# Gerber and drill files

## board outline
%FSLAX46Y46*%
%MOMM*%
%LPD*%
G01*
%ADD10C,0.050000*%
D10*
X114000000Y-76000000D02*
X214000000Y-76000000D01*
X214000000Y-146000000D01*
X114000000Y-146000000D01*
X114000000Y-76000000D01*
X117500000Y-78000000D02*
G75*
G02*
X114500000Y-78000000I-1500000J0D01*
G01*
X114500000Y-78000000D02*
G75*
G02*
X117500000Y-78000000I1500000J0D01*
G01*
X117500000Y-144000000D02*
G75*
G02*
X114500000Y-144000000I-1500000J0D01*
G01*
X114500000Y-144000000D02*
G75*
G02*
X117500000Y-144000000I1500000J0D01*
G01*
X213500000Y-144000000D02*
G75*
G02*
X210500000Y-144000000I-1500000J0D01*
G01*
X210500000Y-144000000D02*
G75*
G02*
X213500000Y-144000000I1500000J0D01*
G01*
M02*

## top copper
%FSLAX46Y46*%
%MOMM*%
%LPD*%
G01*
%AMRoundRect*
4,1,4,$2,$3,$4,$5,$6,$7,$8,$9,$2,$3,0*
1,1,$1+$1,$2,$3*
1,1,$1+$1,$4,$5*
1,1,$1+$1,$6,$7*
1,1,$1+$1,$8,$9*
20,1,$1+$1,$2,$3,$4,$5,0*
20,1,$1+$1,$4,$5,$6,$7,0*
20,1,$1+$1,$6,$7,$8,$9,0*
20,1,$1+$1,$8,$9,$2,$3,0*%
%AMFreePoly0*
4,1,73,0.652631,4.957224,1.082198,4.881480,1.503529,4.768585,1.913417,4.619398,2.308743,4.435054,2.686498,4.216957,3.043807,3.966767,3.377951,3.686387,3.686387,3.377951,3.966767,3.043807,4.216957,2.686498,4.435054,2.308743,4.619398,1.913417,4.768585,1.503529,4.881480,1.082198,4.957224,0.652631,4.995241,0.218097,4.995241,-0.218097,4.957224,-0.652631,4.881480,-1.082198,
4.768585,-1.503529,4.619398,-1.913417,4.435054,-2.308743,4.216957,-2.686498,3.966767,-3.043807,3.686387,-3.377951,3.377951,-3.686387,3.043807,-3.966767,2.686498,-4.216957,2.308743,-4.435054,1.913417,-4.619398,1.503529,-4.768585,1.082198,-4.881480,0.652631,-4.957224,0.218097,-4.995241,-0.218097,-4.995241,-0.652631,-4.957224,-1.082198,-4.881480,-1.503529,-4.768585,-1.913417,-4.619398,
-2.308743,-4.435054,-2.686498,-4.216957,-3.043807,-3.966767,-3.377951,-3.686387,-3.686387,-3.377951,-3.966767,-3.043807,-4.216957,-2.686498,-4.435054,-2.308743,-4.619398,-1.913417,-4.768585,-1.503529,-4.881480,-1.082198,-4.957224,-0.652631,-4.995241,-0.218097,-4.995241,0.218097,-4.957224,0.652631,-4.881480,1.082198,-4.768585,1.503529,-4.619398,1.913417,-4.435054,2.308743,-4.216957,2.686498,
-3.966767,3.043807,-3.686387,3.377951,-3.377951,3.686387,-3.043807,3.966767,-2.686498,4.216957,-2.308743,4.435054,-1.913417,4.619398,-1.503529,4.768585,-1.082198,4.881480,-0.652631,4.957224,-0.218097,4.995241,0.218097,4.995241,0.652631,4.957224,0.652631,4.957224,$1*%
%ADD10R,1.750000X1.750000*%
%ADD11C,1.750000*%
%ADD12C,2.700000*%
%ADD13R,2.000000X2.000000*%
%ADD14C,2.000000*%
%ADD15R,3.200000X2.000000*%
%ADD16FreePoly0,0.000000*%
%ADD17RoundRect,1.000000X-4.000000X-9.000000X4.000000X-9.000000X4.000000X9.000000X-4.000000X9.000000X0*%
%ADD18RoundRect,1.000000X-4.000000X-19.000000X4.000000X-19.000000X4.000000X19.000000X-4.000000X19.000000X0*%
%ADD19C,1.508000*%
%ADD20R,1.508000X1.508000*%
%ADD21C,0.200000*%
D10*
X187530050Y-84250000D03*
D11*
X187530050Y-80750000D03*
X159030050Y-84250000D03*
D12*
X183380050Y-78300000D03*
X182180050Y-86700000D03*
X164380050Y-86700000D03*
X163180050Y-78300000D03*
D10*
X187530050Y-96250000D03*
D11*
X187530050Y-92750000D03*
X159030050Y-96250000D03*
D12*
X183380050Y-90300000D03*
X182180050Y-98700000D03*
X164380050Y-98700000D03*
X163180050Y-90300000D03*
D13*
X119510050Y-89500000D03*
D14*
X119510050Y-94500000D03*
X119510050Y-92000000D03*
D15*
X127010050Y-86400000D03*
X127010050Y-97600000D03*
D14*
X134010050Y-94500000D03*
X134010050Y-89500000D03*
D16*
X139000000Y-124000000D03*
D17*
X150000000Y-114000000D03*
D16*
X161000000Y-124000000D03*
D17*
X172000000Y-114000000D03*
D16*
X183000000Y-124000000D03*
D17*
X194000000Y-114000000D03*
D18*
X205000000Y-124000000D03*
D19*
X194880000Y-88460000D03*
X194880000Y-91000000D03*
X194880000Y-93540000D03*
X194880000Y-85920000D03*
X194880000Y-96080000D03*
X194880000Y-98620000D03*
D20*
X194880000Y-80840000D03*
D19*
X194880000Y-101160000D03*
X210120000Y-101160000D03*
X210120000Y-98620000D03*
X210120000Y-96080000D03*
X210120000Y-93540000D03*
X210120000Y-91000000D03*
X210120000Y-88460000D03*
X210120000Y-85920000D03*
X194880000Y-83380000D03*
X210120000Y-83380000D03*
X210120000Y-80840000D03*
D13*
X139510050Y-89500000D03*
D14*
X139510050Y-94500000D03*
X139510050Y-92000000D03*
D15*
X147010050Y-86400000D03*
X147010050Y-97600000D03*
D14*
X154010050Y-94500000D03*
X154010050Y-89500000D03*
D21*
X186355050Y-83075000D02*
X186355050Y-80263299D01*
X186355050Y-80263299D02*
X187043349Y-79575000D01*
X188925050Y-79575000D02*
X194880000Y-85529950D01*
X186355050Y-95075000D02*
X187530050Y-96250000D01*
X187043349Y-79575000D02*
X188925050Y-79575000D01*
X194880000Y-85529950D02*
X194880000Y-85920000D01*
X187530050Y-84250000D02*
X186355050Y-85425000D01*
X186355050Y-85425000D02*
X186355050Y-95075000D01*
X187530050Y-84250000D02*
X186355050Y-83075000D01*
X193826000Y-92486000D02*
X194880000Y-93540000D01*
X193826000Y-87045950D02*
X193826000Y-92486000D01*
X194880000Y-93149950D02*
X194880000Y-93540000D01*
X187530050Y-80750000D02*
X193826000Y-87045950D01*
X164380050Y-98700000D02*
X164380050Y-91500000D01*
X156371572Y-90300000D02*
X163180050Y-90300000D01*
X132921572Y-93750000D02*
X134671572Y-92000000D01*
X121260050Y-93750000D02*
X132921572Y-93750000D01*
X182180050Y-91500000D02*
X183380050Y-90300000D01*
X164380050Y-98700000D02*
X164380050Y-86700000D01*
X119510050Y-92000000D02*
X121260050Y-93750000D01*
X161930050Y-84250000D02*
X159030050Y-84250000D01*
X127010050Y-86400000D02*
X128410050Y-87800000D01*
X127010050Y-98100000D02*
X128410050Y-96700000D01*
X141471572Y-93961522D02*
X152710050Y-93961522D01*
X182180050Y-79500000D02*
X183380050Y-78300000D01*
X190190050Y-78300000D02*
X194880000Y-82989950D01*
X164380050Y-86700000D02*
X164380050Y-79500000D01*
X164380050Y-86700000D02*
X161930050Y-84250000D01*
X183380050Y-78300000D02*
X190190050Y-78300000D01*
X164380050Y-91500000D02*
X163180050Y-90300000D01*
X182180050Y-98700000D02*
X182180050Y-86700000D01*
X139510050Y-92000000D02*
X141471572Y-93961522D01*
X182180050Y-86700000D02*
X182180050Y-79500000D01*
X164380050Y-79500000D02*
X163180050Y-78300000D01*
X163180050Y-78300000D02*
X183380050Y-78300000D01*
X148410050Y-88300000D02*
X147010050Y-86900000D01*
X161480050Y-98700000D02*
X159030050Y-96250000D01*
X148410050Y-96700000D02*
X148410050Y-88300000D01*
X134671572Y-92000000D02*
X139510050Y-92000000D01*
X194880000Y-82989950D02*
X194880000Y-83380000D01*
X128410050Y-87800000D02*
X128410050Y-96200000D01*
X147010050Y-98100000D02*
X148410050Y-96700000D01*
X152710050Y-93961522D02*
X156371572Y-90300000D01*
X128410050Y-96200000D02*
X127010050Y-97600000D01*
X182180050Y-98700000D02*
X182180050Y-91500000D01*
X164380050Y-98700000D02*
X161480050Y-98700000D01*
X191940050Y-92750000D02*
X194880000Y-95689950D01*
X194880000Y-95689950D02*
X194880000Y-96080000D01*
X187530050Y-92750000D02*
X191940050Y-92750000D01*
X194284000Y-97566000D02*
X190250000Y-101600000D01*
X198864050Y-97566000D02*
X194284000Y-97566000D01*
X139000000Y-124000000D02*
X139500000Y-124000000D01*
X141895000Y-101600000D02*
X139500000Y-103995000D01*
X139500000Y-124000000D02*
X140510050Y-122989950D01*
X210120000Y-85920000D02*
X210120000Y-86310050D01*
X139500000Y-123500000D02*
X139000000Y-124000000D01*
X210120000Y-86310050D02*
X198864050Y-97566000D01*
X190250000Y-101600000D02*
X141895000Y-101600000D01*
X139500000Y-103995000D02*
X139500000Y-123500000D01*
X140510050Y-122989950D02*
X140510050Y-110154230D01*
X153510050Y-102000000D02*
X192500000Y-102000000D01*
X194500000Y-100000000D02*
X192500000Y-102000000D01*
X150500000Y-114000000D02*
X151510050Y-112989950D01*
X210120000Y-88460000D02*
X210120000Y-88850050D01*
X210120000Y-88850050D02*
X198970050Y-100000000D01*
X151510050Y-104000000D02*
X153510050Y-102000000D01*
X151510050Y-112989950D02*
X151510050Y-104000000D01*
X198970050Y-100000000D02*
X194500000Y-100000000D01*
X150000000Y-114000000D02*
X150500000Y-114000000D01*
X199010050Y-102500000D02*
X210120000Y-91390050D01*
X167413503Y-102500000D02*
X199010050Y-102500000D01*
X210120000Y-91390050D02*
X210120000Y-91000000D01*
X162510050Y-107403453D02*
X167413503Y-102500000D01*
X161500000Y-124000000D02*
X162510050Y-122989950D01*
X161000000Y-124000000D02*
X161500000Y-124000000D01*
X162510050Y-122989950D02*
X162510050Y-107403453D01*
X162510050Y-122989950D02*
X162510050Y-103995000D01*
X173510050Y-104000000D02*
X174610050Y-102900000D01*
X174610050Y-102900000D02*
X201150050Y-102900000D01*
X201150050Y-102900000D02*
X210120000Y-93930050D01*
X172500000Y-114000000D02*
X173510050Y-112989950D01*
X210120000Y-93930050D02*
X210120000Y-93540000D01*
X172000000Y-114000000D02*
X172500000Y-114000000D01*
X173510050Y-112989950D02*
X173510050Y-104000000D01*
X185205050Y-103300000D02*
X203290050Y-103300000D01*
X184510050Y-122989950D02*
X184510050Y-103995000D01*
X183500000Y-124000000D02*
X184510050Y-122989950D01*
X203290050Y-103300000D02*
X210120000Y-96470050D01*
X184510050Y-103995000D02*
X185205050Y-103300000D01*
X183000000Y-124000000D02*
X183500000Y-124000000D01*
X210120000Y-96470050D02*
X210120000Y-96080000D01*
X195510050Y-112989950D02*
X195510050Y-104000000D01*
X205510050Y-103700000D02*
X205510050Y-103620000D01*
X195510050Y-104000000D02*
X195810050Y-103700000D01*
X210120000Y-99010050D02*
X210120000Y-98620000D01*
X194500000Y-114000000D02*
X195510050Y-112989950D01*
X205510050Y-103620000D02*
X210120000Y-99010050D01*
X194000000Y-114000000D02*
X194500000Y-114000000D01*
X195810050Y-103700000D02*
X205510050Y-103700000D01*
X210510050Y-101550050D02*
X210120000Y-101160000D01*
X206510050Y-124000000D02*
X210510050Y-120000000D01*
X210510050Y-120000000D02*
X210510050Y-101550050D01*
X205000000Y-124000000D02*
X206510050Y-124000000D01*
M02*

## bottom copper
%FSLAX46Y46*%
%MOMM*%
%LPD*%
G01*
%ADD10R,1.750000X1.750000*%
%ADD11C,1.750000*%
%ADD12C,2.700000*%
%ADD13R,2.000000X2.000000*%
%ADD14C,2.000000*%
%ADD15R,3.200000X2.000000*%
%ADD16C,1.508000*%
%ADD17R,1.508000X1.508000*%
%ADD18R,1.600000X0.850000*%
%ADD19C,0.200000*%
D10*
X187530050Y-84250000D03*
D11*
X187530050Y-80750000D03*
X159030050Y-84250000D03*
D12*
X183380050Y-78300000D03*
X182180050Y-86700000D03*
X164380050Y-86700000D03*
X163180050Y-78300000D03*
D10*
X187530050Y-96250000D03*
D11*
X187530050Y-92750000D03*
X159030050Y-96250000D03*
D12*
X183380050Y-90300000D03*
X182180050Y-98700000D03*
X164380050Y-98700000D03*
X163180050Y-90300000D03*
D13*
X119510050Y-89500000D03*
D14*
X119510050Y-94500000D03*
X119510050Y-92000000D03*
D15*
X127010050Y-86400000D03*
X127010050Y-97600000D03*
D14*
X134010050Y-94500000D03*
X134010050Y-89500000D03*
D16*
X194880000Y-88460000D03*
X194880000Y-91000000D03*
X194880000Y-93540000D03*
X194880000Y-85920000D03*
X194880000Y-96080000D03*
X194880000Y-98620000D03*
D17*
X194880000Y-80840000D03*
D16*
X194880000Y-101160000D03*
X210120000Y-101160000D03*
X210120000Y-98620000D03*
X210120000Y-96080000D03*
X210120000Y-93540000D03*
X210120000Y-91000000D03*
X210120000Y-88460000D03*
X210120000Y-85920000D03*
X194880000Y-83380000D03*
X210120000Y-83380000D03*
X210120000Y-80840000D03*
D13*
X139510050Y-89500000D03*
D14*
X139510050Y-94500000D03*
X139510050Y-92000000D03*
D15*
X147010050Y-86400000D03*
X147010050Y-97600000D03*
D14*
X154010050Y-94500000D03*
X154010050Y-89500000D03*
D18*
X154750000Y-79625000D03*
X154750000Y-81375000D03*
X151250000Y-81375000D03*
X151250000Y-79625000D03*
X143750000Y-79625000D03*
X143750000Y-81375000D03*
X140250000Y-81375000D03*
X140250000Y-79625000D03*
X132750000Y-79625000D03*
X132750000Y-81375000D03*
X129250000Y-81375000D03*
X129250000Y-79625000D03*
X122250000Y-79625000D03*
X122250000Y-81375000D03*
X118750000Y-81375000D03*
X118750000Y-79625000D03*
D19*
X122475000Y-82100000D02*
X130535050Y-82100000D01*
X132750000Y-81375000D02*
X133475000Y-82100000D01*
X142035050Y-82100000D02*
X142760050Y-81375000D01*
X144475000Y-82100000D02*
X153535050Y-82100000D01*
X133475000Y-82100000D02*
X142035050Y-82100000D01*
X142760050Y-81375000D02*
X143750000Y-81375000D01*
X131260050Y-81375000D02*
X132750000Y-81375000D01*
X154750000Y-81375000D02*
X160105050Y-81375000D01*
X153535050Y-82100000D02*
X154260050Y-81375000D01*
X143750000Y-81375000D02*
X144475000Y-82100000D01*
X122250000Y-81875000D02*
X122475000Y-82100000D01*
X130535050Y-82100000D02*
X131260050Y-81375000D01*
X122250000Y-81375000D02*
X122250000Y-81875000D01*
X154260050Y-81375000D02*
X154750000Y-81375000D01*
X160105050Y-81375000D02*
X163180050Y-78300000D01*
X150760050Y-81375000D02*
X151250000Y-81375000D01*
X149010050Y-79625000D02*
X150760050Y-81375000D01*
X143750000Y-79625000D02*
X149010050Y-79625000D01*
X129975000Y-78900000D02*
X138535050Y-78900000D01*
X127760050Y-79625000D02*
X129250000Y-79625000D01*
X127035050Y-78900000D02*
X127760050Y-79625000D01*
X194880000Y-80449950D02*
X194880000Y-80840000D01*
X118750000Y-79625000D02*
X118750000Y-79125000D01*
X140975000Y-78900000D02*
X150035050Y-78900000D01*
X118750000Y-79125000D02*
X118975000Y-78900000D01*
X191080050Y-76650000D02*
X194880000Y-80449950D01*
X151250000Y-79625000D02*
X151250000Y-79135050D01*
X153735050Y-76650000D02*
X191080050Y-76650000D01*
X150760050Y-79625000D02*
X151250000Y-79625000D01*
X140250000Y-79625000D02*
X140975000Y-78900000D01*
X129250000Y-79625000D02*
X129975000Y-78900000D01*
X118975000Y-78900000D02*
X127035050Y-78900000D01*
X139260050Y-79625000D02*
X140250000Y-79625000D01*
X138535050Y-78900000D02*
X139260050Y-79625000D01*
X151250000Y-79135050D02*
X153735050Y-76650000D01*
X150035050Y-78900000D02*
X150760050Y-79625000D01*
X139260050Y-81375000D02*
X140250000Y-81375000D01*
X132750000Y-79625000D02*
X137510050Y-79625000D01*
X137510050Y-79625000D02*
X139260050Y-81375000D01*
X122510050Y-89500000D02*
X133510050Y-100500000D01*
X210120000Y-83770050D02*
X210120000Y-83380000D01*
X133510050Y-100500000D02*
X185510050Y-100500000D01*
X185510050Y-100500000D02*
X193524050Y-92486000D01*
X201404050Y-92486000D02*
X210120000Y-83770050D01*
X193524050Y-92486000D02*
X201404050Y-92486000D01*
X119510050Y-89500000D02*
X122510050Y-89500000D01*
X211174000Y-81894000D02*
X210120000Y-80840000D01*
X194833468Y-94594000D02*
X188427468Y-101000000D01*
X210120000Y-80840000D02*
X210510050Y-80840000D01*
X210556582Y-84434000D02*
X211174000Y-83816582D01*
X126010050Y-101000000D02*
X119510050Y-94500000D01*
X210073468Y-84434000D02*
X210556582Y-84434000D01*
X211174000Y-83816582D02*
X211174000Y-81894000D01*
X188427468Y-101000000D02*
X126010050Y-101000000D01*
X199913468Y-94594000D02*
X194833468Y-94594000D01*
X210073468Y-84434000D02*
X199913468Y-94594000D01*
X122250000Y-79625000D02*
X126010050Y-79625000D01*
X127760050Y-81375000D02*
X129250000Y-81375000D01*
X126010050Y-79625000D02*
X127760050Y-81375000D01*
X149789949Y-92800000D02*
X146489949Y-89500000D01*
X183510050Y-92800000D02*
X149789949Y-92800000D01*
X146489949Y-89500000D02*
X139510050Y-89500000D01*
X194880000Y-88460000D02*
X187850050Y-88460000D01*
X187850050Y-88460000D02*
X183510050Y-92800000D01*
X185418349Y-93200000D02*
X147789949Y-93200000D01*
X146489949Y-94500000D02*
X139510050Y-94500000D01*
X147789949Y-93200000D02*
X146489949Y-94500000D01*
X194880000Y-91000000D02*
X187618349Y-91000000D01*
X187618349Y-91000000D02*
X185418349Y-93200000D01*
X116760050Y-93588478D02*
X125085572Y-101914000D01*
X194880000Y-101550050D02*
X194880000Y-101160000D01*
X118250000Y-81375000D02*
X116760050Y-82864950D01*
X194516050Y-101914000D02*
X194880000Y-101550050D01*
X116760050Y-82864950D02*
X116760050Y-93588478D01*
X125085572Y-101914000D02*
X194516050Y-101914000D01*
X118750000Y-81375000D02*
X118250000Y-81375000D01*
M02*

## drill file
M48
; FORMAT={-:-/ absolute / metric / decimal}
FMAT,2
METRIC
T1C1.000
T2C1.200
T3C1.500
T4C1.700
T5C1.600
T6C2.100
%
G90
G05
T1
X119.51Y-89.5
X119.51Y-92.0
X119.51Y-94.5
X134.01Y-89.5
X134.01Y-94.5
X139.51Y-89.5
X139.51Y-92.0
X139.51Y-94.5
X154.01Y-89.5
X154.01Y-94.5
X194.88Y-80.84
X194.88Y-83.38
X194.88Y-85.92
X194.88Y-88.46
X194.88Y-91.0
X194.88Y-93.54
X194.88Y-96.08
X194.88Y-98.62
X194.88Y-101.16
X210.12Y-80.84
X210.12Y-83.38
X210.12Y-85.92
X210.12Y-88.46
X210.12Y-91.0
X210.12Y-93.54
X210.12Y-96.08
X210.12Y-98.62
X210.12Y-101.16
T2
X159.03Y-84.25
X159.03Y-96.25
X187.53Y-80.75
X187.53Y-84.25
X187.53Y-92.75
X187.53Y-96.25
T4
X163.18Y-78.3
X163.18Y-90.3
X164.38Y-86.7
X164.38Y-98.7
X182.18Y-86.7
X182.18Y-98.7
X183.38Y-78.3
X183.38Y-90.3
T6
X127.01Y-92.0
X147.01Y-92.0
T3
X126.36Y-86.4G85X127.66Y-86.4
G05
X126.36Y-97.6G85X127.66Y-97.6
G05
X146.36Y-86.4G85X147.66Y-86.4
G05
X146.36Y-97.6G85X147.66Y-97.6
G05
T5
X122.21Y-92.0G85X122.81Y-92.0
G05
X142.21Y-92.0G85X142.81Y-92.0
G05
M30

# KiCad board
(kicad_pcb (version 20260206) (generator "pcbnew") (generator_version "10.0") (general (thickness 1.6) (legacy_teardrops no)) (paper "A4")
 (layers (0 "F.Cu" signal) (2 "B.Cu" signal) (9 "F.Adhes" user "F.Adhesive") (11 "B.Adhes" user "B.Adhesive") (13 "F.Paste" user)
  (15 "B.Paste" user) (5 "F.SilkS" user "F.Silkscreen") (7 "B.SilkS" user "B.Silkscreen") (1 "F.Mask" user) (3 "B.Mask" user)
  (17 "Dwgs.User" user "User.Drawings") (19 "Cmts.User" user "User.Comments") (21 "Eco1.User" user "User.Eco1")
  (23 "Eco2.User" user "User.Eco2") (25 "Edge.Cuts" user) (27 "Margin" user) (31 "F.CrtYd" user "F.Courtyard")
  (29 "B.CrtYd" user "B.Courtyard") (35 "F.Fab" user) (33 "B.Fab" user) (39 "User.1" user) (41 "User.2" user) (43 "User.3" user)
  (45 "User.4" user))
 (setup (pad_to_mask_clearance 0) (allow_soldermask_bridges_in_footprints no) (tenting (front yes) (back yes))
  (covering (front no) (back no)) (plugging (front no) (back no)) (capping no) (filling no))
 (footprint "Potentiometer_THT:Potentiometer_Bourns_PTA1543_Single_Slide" (layer "F.Cu") (at 187.53005 84.25 180)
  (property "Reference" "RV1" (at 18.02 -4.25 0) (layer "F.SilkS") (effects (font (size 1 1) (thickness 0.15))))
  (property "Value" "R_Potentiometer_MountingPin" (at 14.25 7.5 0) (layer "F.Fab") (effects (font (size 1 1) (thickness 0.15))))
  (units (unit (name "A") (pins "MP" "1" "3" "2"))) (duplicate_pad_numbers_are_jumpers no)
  (pad "1" thru_hole rect (at 0 0 180) (size 1.75 1.75) (drill 1.2) (layers "*.Cu" "*.Mask") (remove_unused_layers no) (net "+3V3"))
  (pad "2" thru_hole circle (at 0 3.5 180) (size 1.75 1.75) (drill 1.2) (layers "*.Cu" "*.Mask") (remove_unused_layers no) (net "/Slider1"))
  (pad "3" thru_hole circle (at 28.5 0 180) (size 1.75 1.75) (drill 1.2) (layers "*.Cu" "*.Mask") (remove_unused_layers no) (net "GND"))
  (pad "MP" thru_hole circle (at 4.15 5.95 180) (size 2.7 2.7) (drill 1.7) (layers "*.Cu" "*.Mask") (remove_unused_layers no) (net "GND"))
  (pad "MP" thru_hole circle (at 5.35 -2.45 180) (size 2.7 2.7) (drill 1.7) (layers "*.Cu" "*.Mask") (remove_unused_layers no) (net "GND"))
  (pad "MP" thru_hole circle (at 23.15 -2.45 180) (size 2.7 2.7) (drill 1.7) (layers "*.Cu" "*.Mask") (remove_unused_layers no) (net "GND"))
  (pad "MP" thru_hole circle (at 24.35 5.95 180) (size 2.7 2.7) (drill 1.7) (layers "*.Cu" "*.Mask") (remove_unused_layers no) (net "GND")))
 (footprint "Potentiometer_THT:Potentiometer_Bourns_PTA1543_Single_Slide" (layer "F.Cu") (at 187.53005 96.25 180)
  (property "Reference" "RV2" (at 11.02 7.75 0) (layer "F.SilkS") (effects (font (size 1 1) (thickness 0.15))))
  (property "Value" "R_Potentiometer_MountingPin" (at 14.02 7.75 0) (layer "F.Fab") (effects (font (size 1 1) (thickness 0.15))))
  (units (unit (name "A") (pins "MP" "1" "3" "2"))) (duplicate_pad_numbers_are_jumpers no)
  (pad "1" thru_hole rect (at 0 0 180) (size 1.75 1.75) (drill 1.2) (layers "*.Cu" "*.Mask") (remove_unused_layers no) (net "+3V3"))
  (pad "2" thru_hole circle (at 0 3.5 180) (size 1.75 1.75) (drill 1.2) (layers "*.Cu" "*.Mask") (remove_unused_layers no) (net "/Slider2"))
  (pad "3" thru_hole circle (at 28.5 0 180) (size 1.75 1.75) (drill 1.2) (layers "*.Cu" "*.Mask") (remove_unused_layers no) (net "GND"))
  (pad "MP" thru_hole circle (at 4.15 5.95 180) (size 2.7 2.7) (drill 1.7) (layers "*.Cu" "*.Mask") (remove_unused_layers no) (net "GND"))
  (pad "MP" thru_hole circle (at 5.35 -2.45 180) (size 2.7 2.7) (drill 1.7) (layers "*.Cu" "*.Mask") (remove_unused_layers no) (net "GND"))
  (pad "MP" thru_hole circle (at 23.15 -2.45 180) (size 2.7 2.7) (drill 1.7) (layers "*.Cu" "*.Mask") (remove_unused_layers no) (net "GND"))
  (pad "MP" thru_hole circle (at 24.35 5.95 180) (size 2.7 2.7) (drill 1.7) (layers "*.Cu" "*.Mask") (remove_unused_layers no) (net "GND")))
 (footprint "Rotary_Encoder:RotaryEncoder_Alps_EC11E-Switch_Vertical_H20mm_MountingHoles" (layer "F.Cu") (at 119.51005 89.5)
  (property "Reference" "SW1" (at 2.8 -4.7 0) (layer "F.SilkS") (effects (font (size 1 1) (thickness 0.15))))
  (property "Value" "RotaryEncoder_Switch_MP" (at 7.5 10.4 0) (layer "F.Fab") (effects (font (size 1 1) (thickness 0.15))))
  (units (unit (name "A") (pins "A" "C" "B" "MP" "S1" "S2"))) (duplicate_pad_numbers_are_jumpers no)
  (pad "" np_thru_hole oval (at 3 2.5) (size 2.2 1.6) (drill oval 2.2 1.6) (layers "*.Mask"))
  (pad "" np_thru_hole circle (at 7.5 2.5) (size 2.1 2.1) (drill 2.1) (layers "*.Mask"))
  (pad "A" thru_hole rect (at 0 0) (size 2 2) (drill 1) (layers "*.Cu" "*.Mask") (remove_unused_layers no) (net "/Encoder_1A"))
  (pad "B" thru_hole circle (at 0 5) (size 2 2) (drill 1) (layers "*.Cu" "*.Mask") (remove_unused_layers no) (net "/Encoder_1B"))
  (pad "C" thru_hole circle (at 0 2.5) (size 2 2) (drill 1) (layers "*.Cu" "*.Mask") (remove_unused_layers no) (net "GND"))
  (pad "MP" thru_hole rect (at 7.5 -3.1) (size 3.2 2) (drill oval 2.8 1.5) (layers "*.Cu" "*.Mask") (remove_unused_layers no) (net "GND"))
  (pad "MP" thru_hole rect (at 7.5 8.1) (size 3.2 2) (drill oval 2.8 1.5) (layers "*.Cu" "*.Mask") (remove_unused_layers no) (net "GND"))
  (pad "S1" thru_hole circle (at 14.5 5) (size 2 2) (drill 1) (layers "*.Cu" "*.Mask") (remove_unused_layers no)
   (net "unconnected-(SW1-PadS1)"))
  (pad "S2" thru_hole circle (at 14.5 0) (size 2 2) (drill 1) (layers "*.Cu" "*.Mask") (remove_unused_layers no)
   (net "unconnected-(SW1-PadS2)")))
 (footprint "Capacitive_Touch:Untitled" (layer "F.Cu") (at 172 100)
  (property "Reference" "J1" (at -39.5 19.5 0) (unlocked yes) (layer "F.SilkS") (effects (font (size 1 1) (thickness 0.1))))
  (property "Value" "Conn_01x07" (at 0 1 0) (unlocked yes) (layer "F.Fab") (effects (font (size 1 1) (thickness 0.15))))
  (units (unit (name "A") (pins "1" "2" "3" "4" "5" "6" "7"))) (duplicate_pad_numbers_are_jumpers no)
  (pad "1" smd custom (at -33 24) (size 10 10) (layers "F.Cu" "F.Mask") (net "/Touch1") (thermal_bridge_angle 90)
   (options (clearance outline) (anchor circle)) (primitives))
  (pad "2" smd roundrect (at -22 14) (size 10 20) (layers "F.Cu" "F.Mask") (roundrect_rratio 0.1) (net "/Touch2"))
  (pad "3" smd custom (at -11 24) (size 10 10) (layers "F.Cu" "F.Mask") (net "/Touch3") (thermal_bridge_angle 90)
   (options (clearance outline) (anchor circle)) (primitives))
  (pad "4" smd roundrect (at 0 14) (size 10 20) (layers "F.Cu" "F.Mask") (roundrect_rratio 0.1) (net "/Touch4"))
  (pad "5" smd custom (at 11 24) (size 10 10) (layers "F.Cu" "F.Mask") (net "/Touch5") (thermal_bridge_angle 90)
   (options (clearance outline) (anchor circle)) (primitives))
  (pad "6" smd roundrect (at 22 14) (size 10 20) (layers "F.Cu" "F.Mask") (roundrect_rratio 0.1) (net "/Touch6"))
  (pad "7" smd roundrect (at 33 24) (size 10 40) (layers "F.Cu" "F.Mask") (roundrect_rratio 0.1) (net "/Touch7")))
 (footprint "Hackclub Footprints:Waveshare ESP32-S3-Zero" (layer "F.Cu") (at 202.5 91)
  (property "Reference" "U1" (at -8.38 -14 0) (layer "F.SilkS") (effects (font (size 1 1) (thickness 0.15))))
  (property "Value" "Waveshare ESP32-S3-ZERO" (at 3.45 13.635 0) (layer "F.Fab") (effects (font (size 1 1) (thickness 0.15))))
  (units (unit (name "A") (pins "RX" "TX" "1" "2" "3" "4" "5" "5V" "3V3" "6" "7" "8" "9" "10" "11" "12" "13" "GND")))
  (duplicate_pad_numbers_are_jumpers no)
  (pad "1" thru_hole circle (at -7.62 -2.54) (size 1.508 1.508) (drill 1) (layers "*.Cu" "*.Mask") (remove_unused_layers no)
   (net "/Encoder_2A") (solder_mask_margin 0.102))
  (pad "2" thru_hole circle (at -7.62 0) (size 1.508 1.508) (drill 1) (layers "*.Cu" "*.Mask") (remove_unused_layers no) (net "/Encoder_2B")
   (solder_mask_margin 0.102))
  (pad "3" thru_hole circle (at -7.62 2.54) (size 1.508 1.508) (drill 1) (layers "*.Cu" "*.Mask") (remove_unused_layers no) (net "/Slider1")
   (solder_mask_margin 0.102))
  (pad "3V3" thru_hole circle (at -7.62 -5.08) (size 1.508 1.508) (drill 1) (layers "*.Cu" "*.Mask") (remove_unused_layers no) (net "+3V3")
   (solder_mask_margin 0.102))
  (pad "4" thru_hole circle (at -7.62 5.08) (size 1.508 1.508) (drill 1) (layers "*.Cu" "*.Mask") (remove_unused_layers no) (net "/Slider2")
   (solder_mask_margin 0.102))
  (pad "5" thru_hole circle (at -7.62 7.62) (size 1.508 1.508) (drill 1) (layers "*.Cu" "*.Mask") (remove_unused_layers no)
   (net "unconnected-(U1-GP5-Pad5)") (solder_mask_margin 0.102))
  (pad "5V" thru_hole rect (at -7.62 -10.16) (size 1.508 1.508) (drill 1) (layers "*.Cu" "*.Mask") (remove_unused_layers no) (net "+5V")
   (solder_mask_margin 0.102))
  (pad "6" thru_hole circle (at -7.62 10.16) (size 1.508 1.508) (drill 1) (layers "*.Cu" "*.Mask") (remove_unused_layers no) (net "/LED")
   (solder_mask_margin 0.102))
  (pad "7" thru_hole circle (at 7.62 10.16) (size 1.508 1.508) (drill 1) (layers "*.Cu" "*.Mask") (remove_unused_layers no) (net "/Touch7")
   (solder_mask_margin 0.102))
  (pad "8" thru_hole circle (at 7.62 7.62) (size 1.508 1.508) (drill 1) (layers "*.Cu" "*.Mask") (remove_unused_layers no) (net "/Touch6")
   (solder_mask_margin 0.102))
  (pad "9" thru_hole circle (at 7.62 5.08) (size 1.508 1.508) (drill 1) (layers "*.Cu" "*.Mask") (remove_unused_layers no) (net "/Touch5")
   (solder_mask_margin 0.102))
  (pad "10" thru_hole circle (at 7.62 2.54) (size 1.508 1.508) (drill 1) (layers "*.Cu" "*.Mask") (remove_unused_layers no) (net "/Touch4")
   (solder_mask_margin 0.102))
  (pad "11" thru_hole circle (at 7.62 0) (size 1.508 1.508) (drill 1) (layers "*.Cu" "*.Mask") (remove_unused_layers no) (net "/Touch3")
   (solder_mask_margin 0.102))
  (pad "12" thru_hole circle (at 7.62 -2.54) (size 1.508 1.508) (drill 1) (layers "*.Cu" "*.Mask") (remove_unused_layers no) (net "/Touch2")
   (solder_mask_margin 0.102))
  (pad "13" thru_hole circle (at 7.62 -5.08) (size 1.508 1.508) (drill 1) (layers "*.Cu" "*.Mask") (remove_unused_layers no) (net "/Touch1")
   (solder_mask_margin 0.102))
  (pad "GND" thru_hole circle (at -7.62 -7.62) (size 1.508 1.508) (drill 1) (layers "*.Cu" "*.Mask") (remove_unused_layers no) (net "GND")
   (solder_mask_margin 0.102))
  (pad "RX" thru_hole circle (at 7.62 -7.62) (size 1.508 1.508) (drill 1) (layers "*.Cu" "*.Mask") (remove_unused_layers no)
   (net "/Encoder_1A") (solder_mask_margin 0.102))
  (pad "TX" thru_hole circle (at 7.62 -10.16) (size 1.508 1.508) (drill 1) (layers "*.Cu" "*.Mask") (remove_unused_layers no)
   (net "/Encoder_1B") (solder_mask_margin 0.102)))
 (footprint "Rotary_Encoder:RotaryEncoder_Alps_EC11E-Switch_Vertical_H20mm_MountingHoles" (layer "F.Cu") (at 139.51005 89.5)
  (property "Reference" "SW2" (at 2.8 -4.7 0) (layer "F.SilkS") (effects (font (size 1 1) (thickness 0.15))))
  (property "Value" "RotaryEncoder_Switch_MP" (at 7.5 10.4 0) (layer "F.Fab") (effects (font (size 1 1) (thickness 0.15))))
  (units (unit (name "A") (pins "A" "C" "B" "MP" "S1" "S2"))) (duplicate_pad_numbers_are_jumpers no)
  (pad "" np_thru_hole oval (at 3 2.5) (size 2.2 1.6) (drill oval 2.2 1.6) (layers "*.Mask"))
  (pad "" np_thru_hole circle (at 7.5 2.5) (size 2.1 2.1) (drill 2.1) (layers "*.Mask"))
  (pad "A" thru_hole rect (at 0 0) (size 2 2) (drill 1) (layers "*.Cu" "*.Mask") (remove_unused_layers no) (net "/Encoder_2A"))
  (pad "B" thru_hole circle (at 0 5) (size 2 2) (drill 1) (layers "*.Cu" "*.Mask") (remove_unused_layers no) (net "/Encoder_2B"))
  (pad "C" thru_hole circle (at 0 2.5) (size 2 2) (drill 1) (layers "*.Cu" "*.Mask") (remove_unused_layers no) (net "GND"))
  (pad "MP" thru_hole rect (at 7.5 -3.1) (size 3.2 2) (drill oval 2.8 1.5) (layers "*.Cu" "*.Mask") (remove_unused_layers no) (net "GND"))
  (pad "MP" thru_hole rect (at 7.5 8.1) (size 3.2 2) (drill oval 2.8 1.5) (layers "*.Cu" "*.Mask") (remove_unused_layers no) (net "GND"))
  (pad "S1" thru_hole circle (at 14.5 5) (size 2 2) (drill 1) (layers "*.Cu" "*.Mask") (remove_unused_layers no)
   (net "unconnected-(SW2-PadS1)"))
  (pad "S2" thru_hole circle (at 14.5 0) (size 2 2) (drill 1) (layers "*.Cu" "*.Mask") (remove_unused_layers no)
   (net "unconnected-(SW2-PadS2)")))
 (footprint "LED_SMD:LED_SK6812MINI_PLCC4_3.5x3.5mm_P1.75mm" (layer "B.Cu") (at 153 80.5 180)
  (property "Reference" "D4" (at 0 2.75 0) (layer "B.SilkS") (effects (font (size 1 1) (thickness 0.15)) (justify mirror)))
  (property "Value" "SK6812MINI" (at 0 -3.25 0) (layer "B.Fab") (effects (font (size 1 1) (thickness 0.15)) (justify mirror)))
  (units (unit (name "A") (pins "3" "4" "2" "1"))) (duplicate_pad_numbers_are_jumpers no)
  (pad "1" smd rect (at -1.75 0.875 180) (size 1.6 0.85) (layers "B.Cu" "B.Mask" "B.Paste") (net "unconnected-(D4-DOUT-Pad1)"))
  (pad "2" smd rect (at -1.75 -0.875 180) (size 1.6 0.85) (layers "B.Cu" "B.Mask" "B.Paste") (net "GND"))
  (pad "3" smd rect (at 1.75 -0.875 180) (size 1.6 0.85) (layers "B.Cu" "B.Mask" "B.Paste") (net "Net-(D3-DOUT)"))
  (pad "4" smd rect (at 1.75 0.875 180) (size 1.6 0.85) (layers "B.Cu" "B.Mask" "B.Paste") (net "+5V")))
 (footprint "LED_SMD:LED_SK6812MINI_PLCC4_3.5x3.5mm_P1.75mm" (layer "B.Cu") (at 142 80.5 180)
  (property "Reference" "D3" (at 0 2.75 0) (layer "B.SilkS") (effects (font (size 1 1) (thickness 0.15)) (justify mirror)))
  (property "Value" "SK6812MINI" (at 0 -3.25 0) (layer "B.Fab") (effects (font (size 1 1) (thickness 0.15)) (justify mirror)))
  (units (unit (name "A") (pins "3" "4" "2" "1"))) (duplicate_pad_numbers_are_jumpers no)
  (pad "1" smd rect (at -1.75 0.875 180) (size 1.6 0.85) (layers "B.Cu" "B.Mask" "B.Paste") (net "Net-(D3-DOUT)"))
  (pad "2" smd rect (at -1.75 -0.875 180) (size 1.6 0.85) (layers "B.Cu" "B.Mask" "B.Paste") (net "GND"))
  (pad "3" smd rect (at 1.75 -0.875 180) (size 1.6 0.85) (layers "B.Cu" "B.Mask" "B.Paste") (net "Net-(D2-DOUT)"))
  (pad "4" smd rect (at 1.75 0.875 180) (size 1.6 0.85) (layers "B.Cu" "B.Mask" "B.Paste") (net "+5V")))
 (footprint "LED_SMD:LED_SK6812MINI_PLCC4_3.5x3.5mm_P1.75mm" (layer "B.Cu") (at 131 80.5 180)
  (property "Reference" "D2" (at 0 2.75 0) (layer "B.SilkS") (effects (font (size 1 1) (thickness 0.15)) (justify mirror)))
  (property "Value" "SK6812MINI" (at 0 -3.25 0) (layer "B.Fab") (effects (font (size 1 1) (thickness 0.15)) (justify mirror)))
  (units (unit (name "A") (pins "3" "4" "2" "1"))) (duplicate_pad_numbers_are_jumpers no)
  (pad "1" smd rect (at -1.75 0.875 180) (size 1.6 0.85) (layers "B.Cu" "B.Mask" "B.Paste") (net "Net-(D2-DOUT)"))
  (pad "2" smd rect (at -1.75 -0.875 180) (size 1.6 0.85) (layers "B.Cu" "B.Mask" "B.Paste") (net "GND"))
  (pad "3" smd rect (at 1.75 -0.875 180) (size 1.6 0.85) (layers "B.Cu" "B.Mask" "B.Paste") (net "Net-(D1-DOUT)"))
  (pad "4" smd rect (at 1.75 0.875 180) (size 1.6 0.85) (layers "B.Cu" "B.Mask" "B.Paste") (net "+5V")))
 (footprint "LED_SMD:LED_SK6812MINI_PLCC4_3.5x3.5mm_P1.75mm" (layer "B.Cu") (at 120.5 80.5 180)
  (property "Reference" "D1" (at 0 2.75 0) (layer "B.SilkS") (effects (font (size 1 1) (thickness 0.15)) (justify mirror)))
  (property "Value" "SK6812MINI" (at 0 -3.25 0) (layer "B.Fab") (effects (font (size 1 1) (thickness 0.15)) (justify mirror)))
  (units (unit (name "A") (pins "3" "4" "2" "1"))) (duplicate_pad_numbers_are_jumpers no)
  (pad "1" smd rect (at -1.75 0.875 180) (size 1.6 0.85) (layers "B.Cu" "B.Mask" "B.Paste") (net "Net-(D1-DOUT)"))
  (pad "2" smd rect (at -1.75 -0.875 180) (size 1.6 0.85) (layers "B.Cu" "B.Mask" "B.Paste") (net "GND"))
  (pad "3" smd rect (at 1.75 -0.875 180) (size 1.6 0.85) (layers "B.Cu" "B.Mask" "B.Paste") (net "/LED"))
  (pad "4" smd rect (at 1.75 0.875 180) (size 1.6 0.85) (layers "B.Cu" "B.Mask" "B.Paste") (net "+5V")))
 (gr_rect (start 114 76) (end 214 146) (stroke (width 0.05) (type default)) (fill no) (layer "Edge.Cuts"))
 (gr_circle (center 116 78) (end 114.5 78) (stroke (width 0.05) (type default)) (fill no) (layer "Edge.Cuts"))
 (gr_circle (center 116 144) (end 117.5 144) (stroke (width 0.05) (type default)) (fill no) (layer "Edge.Cuts"))
 (gr_circle (center 212 144) (end 213.5 144) (stroke (width 0.05) (type default)) (fill no) (layer "Edge.Cuts"))
 (segment (start 186.35505 83.075) (end 186.35505 80.263299) (width 0.2) (layer "F.Cu") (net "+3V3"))
 (segment (start 186.35505 80.263299) (end 187.043349 79.575) (width 0.2) (layer "F.Cu") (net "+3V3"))
 (segment (start 188.92505 79.575) (end 194.88 85.52995) (width 0.2) (layer "F.Cu") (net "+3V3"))
 (segment (start 186.35505 95.075) (end 187.53005 96.25) (width 0.2) (layer "F.Cu") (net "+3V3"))
 (segment (start 187.043349 79.575) (end 188.92505 79.575) (width 0.2) (layer "F.Cu") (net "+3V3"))
 (segment (start 194.88 85.52995) (end 194.88 85.92) (width 0.2) (layer "F.Cu") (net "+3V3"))
 (segment (start 187.53005 84.25) (end 186.35505 85.425) (width 0.2) (layer "F.Cu") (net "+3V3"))
 (segment (start 186.35505 85.425) (end 186.35505 95.075) (width 0.2) (layer "F.Cu") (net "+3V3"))
 (segment (start 187.53005 84.25) (end 186.35505 83.075) (width 0.2) (layer "F.Cu") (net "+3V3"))
 (segment (start 193.826 92.486) (end 194.88 93.54) (width 0.2) (layer "F.Cu") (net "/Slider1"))
 (segment (start 193.826 87.04595) (end 193.826 92.486) (width 0.2) (layer "F.Cu") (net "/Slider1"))
 (segment (start 194.88 93.14995) (end 194.88 93.54) (width 0.2) (layer "F.Cu") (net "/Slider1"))
 (segment (start 187.53005 80.75) (end 193.826 87.04595) (width 0.2) (layer "F.Cu") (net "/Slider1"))
 (segment (start 164.38005 98.7) (end 164.38005 91.5) (width 0.2) (layer "F.Cu") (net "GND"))
 (segment (start 156.371572 90.3) (end 163.18005 90.3) (width 0.2) (layer "F.Cu") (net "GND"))
 (segment (start 132.921572 93.75) (end 134.671572 92) (width 0.2) (layer "F.Cu") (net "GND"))
 (segment (start 121.26005 93.75) (end 132.921572 93.75) (width 0.2) (layer "F.Cu") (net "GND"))
 (segment (start 182.18005 91.5) (end 183.38005 90.3) (width 0.2) (layer "F.Cu") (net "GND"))
 (segment (start 164.38005 98.7) (end 164.38005 86.7) (width 0.2) (layer "F.Cu") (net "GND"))
 (segment (start 119.51005 92) (end 121.26005 93.75) (width 0.2) (layer "F.Cu") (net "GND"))
 (segment (start 161.93005 84.25) (end 159.03005 84.25) (width 0.2) (layer "F.Cu") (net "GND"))
 (segment (start 127.01005 86.4) (end 128.41005 87.8) (width 0.2) (layer "F.Cu") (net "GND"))
 (segment (start 127.01005 98.1) (end 128.41005 96.7) (width 0.2) (layer "F.Cu") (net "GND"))
 (segment (start 141.471572 93.961522) (end 152.71005 93.961522) (width 0.2) (layer "F.Cu") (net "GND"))
 (segment (start 182.18005 79.5) (end 183.38005 78.3) (width 0.2) (layer "F.Cu") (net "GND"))
 (segment (start 190.19005 78.3) (end 194.88 82.98995) (width 0.2) (layer "F.Cu") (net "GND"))
 (segment (start 164.38005 86.7) (end 164.38005 79.5) (width 0.2) (layer "F.Cu") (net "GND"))
 (segment (start 164.38005 86.7) (end 161.93005 84.25) (width 0.2) (layer "F.Cu") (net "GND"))
 (segment (start 183.38005 78.3) (end 190.19005 78.3) (width 0.2) (layer "F.Cu") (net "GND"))
 (segment (start 164.38005 91.5) (end 163.18005 90.3) (width 0.2) (layer "F.Cu") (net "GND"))
 (segment (start 182.18005 98.7) (end 182.18005 86.7) (width 0.2) (layer "F.Cu") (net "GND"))
 (segment (start 139.51005 92) (end 141.471572 93.961522) (width 0.2) (layer "F.Cu") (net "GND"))
 (segment (start 182.18005 86.7) (end 182.18005 79.5) (width 0.2) (layer "F.Cu") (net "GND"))
 (segment (start 164.38005 79.5) (end 163.18005 78.3) (width 0.2) (layer "F.Cu") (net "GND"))
 (segment (start 163.18005 78.3) (end 183.38005 78.3) (width 0.2) (layer "F.Cu") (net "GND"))
 (segment (start 148.41005 88.3) (end 147.01005 86.9) (width 0.2) (layer "F.Cu") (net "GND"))
 (segment (start 161.48005 98.7) (end 159.03005 96.25) (width 0.2) (layer "F.Cu") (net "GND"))
 (segment (start 148.41005 96.7) (end 148.41005 88.3) (width 0.2) (layer "F.Cu") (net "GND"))
 (segment (start 134.671572 92) (end 139.51005 92) (width 0.2) (layer "F.Cu") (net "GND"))
 (segment (start 194.88 82.98995) (end 194.88 83.38) (width 0.2) (layer "F.Cu") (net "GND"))
 (segment (start 128.41005 87.8) (end 128.41005 96.2) (width 0.2) (layer "F.Cu") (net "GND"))
 (segment (start 147.01005 98.1) (end 148.41005 96.7) (width 0.2) (layer "F.Cu") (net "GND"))
 (segment (start 152.71005 93.961522) (end 156.371572 90.3) (width 0.2) (layer "F.Cu") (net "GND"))
 (segment (start 128.41005 96.2) (end 127.01005 97.6) (width 0.2) (layer "F.Cu") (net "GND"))
 (segment (start 182.18005 98.7) (end 182.18005 91.5) (width 0.2) (layer "F.Cu") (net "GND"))
 (segment (start 164.38005 98.7) (end 161.48005 98.7) (width 0.2) (layer "F.Cu") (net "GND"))
 (segment (start 122.475 82.1) (end 130.53505 82.1) (width 0.2) (layer "B.Cu") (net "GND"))
 (segment (start 132.75 81.375) (end 133.475 82.1) (width 0.2) (layer "B.Cu") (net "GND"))
 (segment (start 142.03505 82.1) (end 142.76005 81.375) (width 0.2) (layer "B.Cu") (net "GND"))
 (segment (start 144.475 82.1) (end 153.53505 82.1) (width 0.2) (layer "B.Cu") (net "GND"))
 (segment (start 133.475 82.1) (end 142.03505 82.1) (width 0.2) (layer "B.Cu") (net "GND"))
 (segment (start 142.76005 81.375) (end 143.75 81.375) (width 0.2) (layer "B.Cu") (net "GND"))
 (segment (start 131.26005 81.375) (end 132.75 81.375) (width 0.2) (layer "B.Cu") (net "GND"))
 (segment (start 154.75 81.375) (end 160.10505 81.375) (width 0.2) (layer "B.Cu") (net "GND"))
 (segment (start 153.53505 82.1) (end 154.26005 81.375) (width 0.2) (layer "B.Cu") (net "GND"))
 (segment (start 143.75 81.375) (end 144.475 82.1) (width 0.2) (layer "B.Cu") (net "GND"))
 (segment (start 122.25 81.875) (end 122.475 82.1) (width 0.2) (layer "B.Cu") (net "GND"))
 (segment (start 130.53505 82.1) (end 131.26005 81.375) (width 0.2) (layer "B.Cu") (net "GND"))
 (segment (start 122.25 81.375) (end 122.25 81.875) (width 0.2) (layer "B.Cu") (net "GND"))
 (segment (start 154.26005 81.375) (end 154.75 81.375) (width 0.2) (layer "B.Cu") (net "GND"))
 (segment (start 160.10505 81.375) (end 163.18005 78.3) (width 0.2) (layer "B.Cu") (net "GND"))
 (segment (start 150.76005 81.375) (end 151.25 81.375) (width 0.2) (layer "B.Cu") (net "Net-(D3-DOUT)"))
 (segment (start 149.01005 79.625) (end 150.76005 81.375) (width 0.2) (layer "B.Cu") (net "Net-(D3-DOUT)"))
 (segment (start 143.75 79.625) (end 149.01005 79.625) (width 0.2) (layer "B.Cu") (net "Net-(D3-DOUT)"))
 (segment (start 129.975 78.9) (end 138.53505 78.9) (width 0.2) (layer "B.Cu") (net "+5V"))
 (segment (start 127.76005 79.625) (end 129.25 79.625) (width 0.2) (layer "B.Cu") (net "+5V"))
 (segment (start 127.03505 78.9) (end 127.76005 79.625) (width 0.2) (layer "B.Cu") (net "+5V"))
 (segment (start 194.88 80.44995) (end 194.88 80.84) (width 0.2) (layer "B.Cu") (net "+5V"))
 (segment (start 118.75 79.625) (end 118.75 79.125) (width 0.2) (layer "B.Cu") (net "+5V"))
 (segment (start 140.975 78.9) (end 150.03505 78.9) (width 0.2) (layer "B.Cu") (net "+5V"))
 (segment (start 118.75 79.125) (end 118.975 78.9) (width 0.2) (layer "B.Cu") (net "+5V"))
 (segment (start 191.08005 76.65) (end 194.88 80.44995) (width 0.2) (layer "B.Cu") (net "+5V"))
 (segment (start 151.25 79.625) (end 151.25 79.13505) (width 0.2) (layer "B.Cu") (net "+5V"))
 (segment (start 153.73505 76.65) (end 191.08005 76.65) (width 0.2) (layer "B.Cu") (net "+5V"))
 (segment (start 150.76005 79.625) (end 151.25 79.625) (width 0.2) (layer "B.Cu") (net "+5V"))
 (segment (start 140.25 79.625) (end 140.975 78.9) (width 0.2) (layer "B.Cu") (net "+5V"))
 (segment (start 129.25 79.625) (end 129.975 78.9) (width 0.2) (layer "B.Cu") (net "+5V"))
 (segment (start 118.975 78.9) (end 127.03505 78.9) (width 0.2) (layer "B.Cu") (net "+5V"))
 (segment (start 139.26005 79.625) (end 140.25 79.625) (width 0.2) (layer "B.Cu") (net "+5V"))
 (segment (start 138.53505 78.9) (end 139.26005 79.625) (width 0.2) (layer "B.Cu") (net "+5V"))
 (segment (start 151.25 79.13505) (end 153.73505 76.65) (width 0.2) (layer "B.Cu") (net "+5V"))
 (segment (start 150.03505 78.9) (end 150.76005 79.625) (width 0.2) (layer "B.Cu") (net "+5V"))
 (segment (start 139.26005 81.375) (end 140.25 81.375) (width 0.2) (layer "B.Cu") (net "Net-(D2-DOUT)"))
 (segment (start 132.75 79.625) (end 137.51005 79.625) (width 0.2) (layer "B.Cu") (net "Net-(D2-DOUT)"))
 (segment (start 137.51005 79.625) (end 139.26005 81.375) (width 0.2) (layer "B.Cu") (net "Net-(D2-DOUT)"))
 (segment (start 191.94005 92.75) (end 194.88 95.68995) (width 0.2) (layer "F.Cu") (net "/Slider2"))
 (segment (start 194.88 95.68995) (end 194.88 96.08) (width 0.2) (layer "F.Cu") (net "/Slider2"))
 (segment (start 187.53005 92.75) (end 191.94005 92.75) (width 0.2) (layer "F.Cu") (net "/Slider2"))
 (segment (start 122.51005 89.5) (end 133.51005 100.5) (width 0.2) (layer "B.Cu") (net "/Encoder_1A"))
 (segment (start 210.12 83.77005) (end 210.12 83.38) (width 0.2) (layer "B.Cu") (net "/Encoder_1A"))
 (segment (start 133.51005 100.5) (end 185.51005 100.5) (width 0.2) (layer "B.Cu") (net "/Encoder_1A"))
 (segment (start 185.51005 100.5) (end 193.52405 92.486) (width 0.2) (layer "B.Cu") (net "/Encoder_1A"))
 (segment (start 201.40405 92.486) (end 210.12 83.77005) (width 0.2) (layer "B.Cu") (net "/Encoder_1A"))
 (segment (start 193.52405 92.486) (end 201.40405 92.486) (width 0.2) (layer "B.Cu") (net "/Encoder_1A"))
 (segment (start 119.51005 89.5) (end 122.51005 89.5) (width 0.2) (layer "B.Cu") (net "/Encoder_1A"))
 (segment (start 211.174 81.894) (end 210.12 80.84) (width 0.2) (layer "B.Cu") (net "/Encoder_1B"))
 (segment (start 194.833468 94.594) (end 188.427468 101) (width 0.2) (layer "B.Cu") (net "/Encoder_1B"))
 (segment (start 210.12 80.84) (end 210.51005 80.84) (width 0.2) (layer "B.Cu") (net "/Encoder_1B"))
 (segment (start 210.556582 84.434) (end 211.174 83.816582) (width 0.2) (layer "B.Cu") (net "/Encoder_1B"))
 (segment (start 126.01005 101) (end 119.51005 94.5) (width 0.2) (layer "B.Cu") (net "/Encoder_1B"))
 (segment (start 210.073468 84.434) (end 210.556582 84.434) (width 0.2) (layer "B.Cu") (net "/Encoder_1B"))
 (segment (start 211.174 83.816582) (end 211.174 81.894) (width 0.2) (layer "B.Cu") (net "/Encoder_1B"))
 (segment (start 188.427468 101) (end 126.01005 101) (width 0.2) (layer "B.Cu") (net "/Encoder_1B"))
 (segment (start 199.913468 94.594) (end 194.833468 94.594) (width 0.2) (layer "B.Cu") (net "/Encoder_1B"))
 (segment (start 210.073468 84.434) (end 199.913468 94.594) (width 0.2) (layer "B.Cu") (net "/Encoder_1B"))
 (segment (start 122.25 79.625) (end 126.01005 79.625) (width 0.2) (layer "B.Cu") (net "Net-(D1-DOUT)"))
 (segment (start 127.76005 81.375) (end 129.25 81.375) (width 0.2) (layer "B.Cu") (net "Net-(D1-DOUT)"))
 (segment (start 126.01005 79.625) (end 127.76005 81.375) (width 0.2) (layer "B.Cu") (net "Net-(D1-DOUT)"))
 (segment (start 194.284 97.566) (end 190.25 101.6) (width 0.2) (layer "F.Cu") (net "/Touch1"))
 (segment (start 198.86405 97.566) (end 194.284 97.566) (width 0.2) (layer "F.Cu") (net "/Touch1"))
 (segment (start 139 124) (end 139.5 124) (width 0.2) (layer "F.Cu") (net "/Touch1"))
 (segment (start 141.895 101.6) (end 139.5 103.995) (width 0.2) (layer "F.Cu") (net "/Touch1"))
 (segment (start 139.5 124) (end 140.51005 122.98995) (width 0.2) (layer "F.Cu") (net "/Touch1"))
 (segment (start 210.12 85.92) (end 210.12 86.31005) (width 0.2) (layer "F.Cu") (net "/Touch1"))
 (segment (start 139.5 123.5) (end 139 124) (width 0.2) (layer "F.Cu") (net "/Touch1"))
 (segment (start 210.12 86.31005) (end 198.86405 97.566) (width 0.2) (layer "F.Cu") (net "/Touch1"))
 (segment (start 190.25 101.6) (end 141.895 101.6) (width 0.2) (layer "F.Cu") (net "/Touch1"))
 (segment (start 139.5 103.995) (end 139.5 123.5) (width 0.2) (layer "F.Cu") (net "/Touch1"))
 (segment (start 140.51005 122.98995) (end 140.51005 110.15423) (width 0.2) (layer "F.Cu") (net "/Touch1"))
 (segment (start 153.51005 102) (end 192.5 102) (width 0.2) (layer "F.Cu") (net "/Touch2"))
 (segment (start 194.5 100) (end 192.5 102) (width 0.2) (layer "F.Cu") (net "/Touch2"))
 (segment (start 150.5 114) (end 151.51005 112.98995) (width 0.2) (layer "F.Cu") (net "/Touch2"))
 (segment (start 210.12 88.46) (end 210.12 88.85005) (width 0.2) (layer "F.Cu") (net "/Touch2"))
 (segment (start 210.12 88.85005) (end 198.97005 100) (width 0.2) (layer "F.Cu") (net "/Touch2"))
 (segment (start 151.51005 104) (end 153.51005 102) (width 0.2) (layer "F.Cu") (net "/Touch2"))
 (segment (start 151.51005 112.98995) (end 151.51005 104) (width 0.2) (layer "F.Cu") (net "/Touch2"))
 (segment (start 198.97005 100) (end 194.5 100) (width 0.2) (layer "F.Cu") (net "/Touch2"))
 (segment (start 150 114) (end 150.5 114) (width 0.2) (layer "F.Cu") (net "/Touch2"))
 (segment (start 199.01005 102.5) (end 210.12 91.39005) (width 0.2) (layer "F.Cu") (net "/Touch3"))
 (segment (start 167.413503 102.5) (end 199.01005 102.5) (width 0.2) (layer "F.Cu") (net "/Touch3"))
 (segment (start 210.12 91.39005) (end 210.12 91) (width 0.2) (layer "F.Cu") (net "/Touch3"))
 (segment (start 162.51005 107.403453) (end 167.413503 102.5) (width 0.2) (layer "F.Cu") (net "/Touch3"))
 (segment (start 161.5 124) (end 162.51005 122.98995) (width 0.2) (layer "F.Cu") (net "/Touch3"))
 (segment (start 161 124) (end 161.5 124) (width 0.2) (layer "F.Cu") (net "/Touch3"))
 (segment (start 162.51005 122.98995) (end 162.51005 107.403453) (width 0.2) (layer "F.Cu") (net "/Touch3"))
 (segment (start 162.51005 122.98995) (end 162.51005 103.995) (width 0.2) (layer "F.Cu") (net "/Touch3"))
 (segment (start 173.51005 104) (end 174.61005 102.9) (width 0.2) (layer "F.Cu") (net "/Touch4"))
 (segment (start 174.61005 102.9) (end 201.15005 102.9) (width 0.2) (layer "F.Cu") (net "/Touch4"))
 (segment (start 201.15005 102.9) (end 210.12 93.93005) (width 0.2) (layer "F.Cu") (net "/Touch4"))
 (segment (start 172.5 114) (end 173.51005 112.98995) (width 0.2) (layer "F.Cu") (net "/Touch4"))
 (segment (start 210.12 93.93005) (end 210.12 93.54) (width 0.2) (layer "F.Cu") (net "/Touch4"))
 (segment (start 172 114) (end 172.5 114) (width 0.2) (layer "F.Cu") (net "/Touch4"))
 (segment (start 173.51005 112.98995) (end 173.51005 104) (width 0.2) (layer "F.Cu") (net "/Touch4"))
 (segment (start 185.20505 103.3) (end 203.29005 103.3) (width 0.2) (layer "F.Cu") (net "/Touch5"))
 (segment (start 184.51005 122.98995) (end 184.51005 103.995) (width 0.2) (layer "F.Cu") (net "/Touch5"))
 (segment (start 183.5 124) (end 184.51005 122.98995) (width 0.2) (layer "F.Cu") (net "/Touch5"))
 (segment (start 203.29005 103.3) (end 210.12 96.47005) (width 0.2) (layer "F.Cu") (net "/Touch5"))
 (segment (start 184.51005 103.995) (end 185.20505 103.3) (width 0.2) (layer "F.Cu") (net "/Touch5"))
 (segment (start 183 124) (end 183.5 124) (width 0.2) (layer "F.Cu") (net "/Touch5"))
 (segment (start 210.12 96.47005) (end 210.12 96.08) (width 0.2) (layer "F.Cu") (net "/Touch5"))
 (segment (start 195.51005 112.98995) (end 195.51005 104) (width 0.2) (layer "F.Cu") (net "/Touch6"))
 (segment (start 205.51005 103.7) (end 205.51005 103.62) (width 0.2) (layer "F.Cu") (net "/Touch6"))
 (segment (start 195.51005 104) (end 195.81005 103.7) (width 0.2) (layer "F.Cu") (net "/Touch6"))
 (segment (start 210.12 99.01005) (end 210.12 98.62) (width 0.2) (layer "F.Cu") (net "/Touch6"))
 (segment (start 194.5 114) (end 195.51005 112.98995) (width 0.2) (layer "F.Cu") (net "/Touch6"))
 (segment (start 205.51005 103.62) (end 210.12 99.01005) (width 0.2) (layer "F.Cu") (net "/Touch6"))
 (segment (start 194 114) (end 194.5 114) (width 0.2) (layer "F.Cu") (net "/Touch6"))
 (segment (start 195.81005 103.7) (end 205.51005 103.7) (width 0.2) (layer "F.Cu") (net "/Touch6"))
 (segment (start 210.51005 101.55005) (end 210.12 101.16) (width 0.2) (layer "F.Cu") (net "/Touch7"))
 (segment (start 206.51005 124) (end 210.51005 120) (width 0.2) (layer "F.Cu") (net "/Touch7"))
 (segment (start 210.51005 120) (end 210.51005 101.55005) (width 0.2) (layer "F.Cu") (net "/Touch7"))
 (segment (start 205 124) (end 206.51005 124) (width 0.2) (layer "F.Cu") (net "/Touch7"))
 (segment (start 149.789949 92.8) (end 146.489949 89.5) (width 0.2) (layer "B.Cu") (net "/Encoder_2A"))
 (segment (start 183.51005 92.8) (end 149.789949 92.8) (width 0.2) (layer "B.Cu") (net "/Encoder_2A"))
 (segment (start 146.489949 89.5) (end 139.51005 89.5) (width 0.2) (layer "B.Cu") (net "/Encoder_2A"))
 (segment (start 194.88 88.46) (end 187.85005 88.46) (width 0.2) (layer "B.Cu") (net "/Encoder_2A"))
 (segment (start 187.85005 88.46) (end 183.51005 92.8) (width 0.2) (layer "B.Cu") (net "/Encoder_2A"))
 (segment (start 185.418349 93.2) (end 147.789949 93.2) (width 0.2) (layer "B.Cu") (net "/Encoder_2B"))
 (segment (start 146.489949 94.5) (end 139.51005 94.5) (width 0.2) (layer "B.Cu") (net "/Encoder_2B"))
 (segment (start 147.789949 93.2) (end 146.489949 94.5) (width 0.2) (layer "B.Cu") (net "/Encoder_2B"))
 (segment (start 194.88 91) (end 187.618349 91) (width 0.2) (layer "B.Cu") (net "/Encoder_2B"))
 (segment (start 187.618349 91) (end 185.418349 93.2) (width 0.2) (layer "B.Cu") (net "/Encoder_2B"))
 (segment (start 116.76005 93.588478) (end 125.085572 101.914) (width 0.2) (layer "B.Cu") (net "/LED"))
 (segment (start 194.88 101.55005) (end 194.88 101.16) (width 0.2) (layer "B.Cu") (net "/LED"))
 (segment (start 118.25 81.375) (end 116.76005 82.86495) (width 0.2) (layer "B.Cu") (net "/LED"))
 (segment (start 194.51605 101.914) (end 194.88 101.55005) (width 0.2) (layer "B.Cu") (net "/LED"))
 (segment (start 116.76005 82.86495) (end 116.76005 93.588478) (width 0.2) (layer "B.Cu") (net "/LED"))
 (segment (start 125.085572 101.914) (end 194.51605 101.914) (width 0.2) (layer "B.Cu") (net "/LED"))
 (segment (start 118.75 81.375) (end 118.25 81.375) (width 0.2) (layer "B.Cu") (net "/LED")))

